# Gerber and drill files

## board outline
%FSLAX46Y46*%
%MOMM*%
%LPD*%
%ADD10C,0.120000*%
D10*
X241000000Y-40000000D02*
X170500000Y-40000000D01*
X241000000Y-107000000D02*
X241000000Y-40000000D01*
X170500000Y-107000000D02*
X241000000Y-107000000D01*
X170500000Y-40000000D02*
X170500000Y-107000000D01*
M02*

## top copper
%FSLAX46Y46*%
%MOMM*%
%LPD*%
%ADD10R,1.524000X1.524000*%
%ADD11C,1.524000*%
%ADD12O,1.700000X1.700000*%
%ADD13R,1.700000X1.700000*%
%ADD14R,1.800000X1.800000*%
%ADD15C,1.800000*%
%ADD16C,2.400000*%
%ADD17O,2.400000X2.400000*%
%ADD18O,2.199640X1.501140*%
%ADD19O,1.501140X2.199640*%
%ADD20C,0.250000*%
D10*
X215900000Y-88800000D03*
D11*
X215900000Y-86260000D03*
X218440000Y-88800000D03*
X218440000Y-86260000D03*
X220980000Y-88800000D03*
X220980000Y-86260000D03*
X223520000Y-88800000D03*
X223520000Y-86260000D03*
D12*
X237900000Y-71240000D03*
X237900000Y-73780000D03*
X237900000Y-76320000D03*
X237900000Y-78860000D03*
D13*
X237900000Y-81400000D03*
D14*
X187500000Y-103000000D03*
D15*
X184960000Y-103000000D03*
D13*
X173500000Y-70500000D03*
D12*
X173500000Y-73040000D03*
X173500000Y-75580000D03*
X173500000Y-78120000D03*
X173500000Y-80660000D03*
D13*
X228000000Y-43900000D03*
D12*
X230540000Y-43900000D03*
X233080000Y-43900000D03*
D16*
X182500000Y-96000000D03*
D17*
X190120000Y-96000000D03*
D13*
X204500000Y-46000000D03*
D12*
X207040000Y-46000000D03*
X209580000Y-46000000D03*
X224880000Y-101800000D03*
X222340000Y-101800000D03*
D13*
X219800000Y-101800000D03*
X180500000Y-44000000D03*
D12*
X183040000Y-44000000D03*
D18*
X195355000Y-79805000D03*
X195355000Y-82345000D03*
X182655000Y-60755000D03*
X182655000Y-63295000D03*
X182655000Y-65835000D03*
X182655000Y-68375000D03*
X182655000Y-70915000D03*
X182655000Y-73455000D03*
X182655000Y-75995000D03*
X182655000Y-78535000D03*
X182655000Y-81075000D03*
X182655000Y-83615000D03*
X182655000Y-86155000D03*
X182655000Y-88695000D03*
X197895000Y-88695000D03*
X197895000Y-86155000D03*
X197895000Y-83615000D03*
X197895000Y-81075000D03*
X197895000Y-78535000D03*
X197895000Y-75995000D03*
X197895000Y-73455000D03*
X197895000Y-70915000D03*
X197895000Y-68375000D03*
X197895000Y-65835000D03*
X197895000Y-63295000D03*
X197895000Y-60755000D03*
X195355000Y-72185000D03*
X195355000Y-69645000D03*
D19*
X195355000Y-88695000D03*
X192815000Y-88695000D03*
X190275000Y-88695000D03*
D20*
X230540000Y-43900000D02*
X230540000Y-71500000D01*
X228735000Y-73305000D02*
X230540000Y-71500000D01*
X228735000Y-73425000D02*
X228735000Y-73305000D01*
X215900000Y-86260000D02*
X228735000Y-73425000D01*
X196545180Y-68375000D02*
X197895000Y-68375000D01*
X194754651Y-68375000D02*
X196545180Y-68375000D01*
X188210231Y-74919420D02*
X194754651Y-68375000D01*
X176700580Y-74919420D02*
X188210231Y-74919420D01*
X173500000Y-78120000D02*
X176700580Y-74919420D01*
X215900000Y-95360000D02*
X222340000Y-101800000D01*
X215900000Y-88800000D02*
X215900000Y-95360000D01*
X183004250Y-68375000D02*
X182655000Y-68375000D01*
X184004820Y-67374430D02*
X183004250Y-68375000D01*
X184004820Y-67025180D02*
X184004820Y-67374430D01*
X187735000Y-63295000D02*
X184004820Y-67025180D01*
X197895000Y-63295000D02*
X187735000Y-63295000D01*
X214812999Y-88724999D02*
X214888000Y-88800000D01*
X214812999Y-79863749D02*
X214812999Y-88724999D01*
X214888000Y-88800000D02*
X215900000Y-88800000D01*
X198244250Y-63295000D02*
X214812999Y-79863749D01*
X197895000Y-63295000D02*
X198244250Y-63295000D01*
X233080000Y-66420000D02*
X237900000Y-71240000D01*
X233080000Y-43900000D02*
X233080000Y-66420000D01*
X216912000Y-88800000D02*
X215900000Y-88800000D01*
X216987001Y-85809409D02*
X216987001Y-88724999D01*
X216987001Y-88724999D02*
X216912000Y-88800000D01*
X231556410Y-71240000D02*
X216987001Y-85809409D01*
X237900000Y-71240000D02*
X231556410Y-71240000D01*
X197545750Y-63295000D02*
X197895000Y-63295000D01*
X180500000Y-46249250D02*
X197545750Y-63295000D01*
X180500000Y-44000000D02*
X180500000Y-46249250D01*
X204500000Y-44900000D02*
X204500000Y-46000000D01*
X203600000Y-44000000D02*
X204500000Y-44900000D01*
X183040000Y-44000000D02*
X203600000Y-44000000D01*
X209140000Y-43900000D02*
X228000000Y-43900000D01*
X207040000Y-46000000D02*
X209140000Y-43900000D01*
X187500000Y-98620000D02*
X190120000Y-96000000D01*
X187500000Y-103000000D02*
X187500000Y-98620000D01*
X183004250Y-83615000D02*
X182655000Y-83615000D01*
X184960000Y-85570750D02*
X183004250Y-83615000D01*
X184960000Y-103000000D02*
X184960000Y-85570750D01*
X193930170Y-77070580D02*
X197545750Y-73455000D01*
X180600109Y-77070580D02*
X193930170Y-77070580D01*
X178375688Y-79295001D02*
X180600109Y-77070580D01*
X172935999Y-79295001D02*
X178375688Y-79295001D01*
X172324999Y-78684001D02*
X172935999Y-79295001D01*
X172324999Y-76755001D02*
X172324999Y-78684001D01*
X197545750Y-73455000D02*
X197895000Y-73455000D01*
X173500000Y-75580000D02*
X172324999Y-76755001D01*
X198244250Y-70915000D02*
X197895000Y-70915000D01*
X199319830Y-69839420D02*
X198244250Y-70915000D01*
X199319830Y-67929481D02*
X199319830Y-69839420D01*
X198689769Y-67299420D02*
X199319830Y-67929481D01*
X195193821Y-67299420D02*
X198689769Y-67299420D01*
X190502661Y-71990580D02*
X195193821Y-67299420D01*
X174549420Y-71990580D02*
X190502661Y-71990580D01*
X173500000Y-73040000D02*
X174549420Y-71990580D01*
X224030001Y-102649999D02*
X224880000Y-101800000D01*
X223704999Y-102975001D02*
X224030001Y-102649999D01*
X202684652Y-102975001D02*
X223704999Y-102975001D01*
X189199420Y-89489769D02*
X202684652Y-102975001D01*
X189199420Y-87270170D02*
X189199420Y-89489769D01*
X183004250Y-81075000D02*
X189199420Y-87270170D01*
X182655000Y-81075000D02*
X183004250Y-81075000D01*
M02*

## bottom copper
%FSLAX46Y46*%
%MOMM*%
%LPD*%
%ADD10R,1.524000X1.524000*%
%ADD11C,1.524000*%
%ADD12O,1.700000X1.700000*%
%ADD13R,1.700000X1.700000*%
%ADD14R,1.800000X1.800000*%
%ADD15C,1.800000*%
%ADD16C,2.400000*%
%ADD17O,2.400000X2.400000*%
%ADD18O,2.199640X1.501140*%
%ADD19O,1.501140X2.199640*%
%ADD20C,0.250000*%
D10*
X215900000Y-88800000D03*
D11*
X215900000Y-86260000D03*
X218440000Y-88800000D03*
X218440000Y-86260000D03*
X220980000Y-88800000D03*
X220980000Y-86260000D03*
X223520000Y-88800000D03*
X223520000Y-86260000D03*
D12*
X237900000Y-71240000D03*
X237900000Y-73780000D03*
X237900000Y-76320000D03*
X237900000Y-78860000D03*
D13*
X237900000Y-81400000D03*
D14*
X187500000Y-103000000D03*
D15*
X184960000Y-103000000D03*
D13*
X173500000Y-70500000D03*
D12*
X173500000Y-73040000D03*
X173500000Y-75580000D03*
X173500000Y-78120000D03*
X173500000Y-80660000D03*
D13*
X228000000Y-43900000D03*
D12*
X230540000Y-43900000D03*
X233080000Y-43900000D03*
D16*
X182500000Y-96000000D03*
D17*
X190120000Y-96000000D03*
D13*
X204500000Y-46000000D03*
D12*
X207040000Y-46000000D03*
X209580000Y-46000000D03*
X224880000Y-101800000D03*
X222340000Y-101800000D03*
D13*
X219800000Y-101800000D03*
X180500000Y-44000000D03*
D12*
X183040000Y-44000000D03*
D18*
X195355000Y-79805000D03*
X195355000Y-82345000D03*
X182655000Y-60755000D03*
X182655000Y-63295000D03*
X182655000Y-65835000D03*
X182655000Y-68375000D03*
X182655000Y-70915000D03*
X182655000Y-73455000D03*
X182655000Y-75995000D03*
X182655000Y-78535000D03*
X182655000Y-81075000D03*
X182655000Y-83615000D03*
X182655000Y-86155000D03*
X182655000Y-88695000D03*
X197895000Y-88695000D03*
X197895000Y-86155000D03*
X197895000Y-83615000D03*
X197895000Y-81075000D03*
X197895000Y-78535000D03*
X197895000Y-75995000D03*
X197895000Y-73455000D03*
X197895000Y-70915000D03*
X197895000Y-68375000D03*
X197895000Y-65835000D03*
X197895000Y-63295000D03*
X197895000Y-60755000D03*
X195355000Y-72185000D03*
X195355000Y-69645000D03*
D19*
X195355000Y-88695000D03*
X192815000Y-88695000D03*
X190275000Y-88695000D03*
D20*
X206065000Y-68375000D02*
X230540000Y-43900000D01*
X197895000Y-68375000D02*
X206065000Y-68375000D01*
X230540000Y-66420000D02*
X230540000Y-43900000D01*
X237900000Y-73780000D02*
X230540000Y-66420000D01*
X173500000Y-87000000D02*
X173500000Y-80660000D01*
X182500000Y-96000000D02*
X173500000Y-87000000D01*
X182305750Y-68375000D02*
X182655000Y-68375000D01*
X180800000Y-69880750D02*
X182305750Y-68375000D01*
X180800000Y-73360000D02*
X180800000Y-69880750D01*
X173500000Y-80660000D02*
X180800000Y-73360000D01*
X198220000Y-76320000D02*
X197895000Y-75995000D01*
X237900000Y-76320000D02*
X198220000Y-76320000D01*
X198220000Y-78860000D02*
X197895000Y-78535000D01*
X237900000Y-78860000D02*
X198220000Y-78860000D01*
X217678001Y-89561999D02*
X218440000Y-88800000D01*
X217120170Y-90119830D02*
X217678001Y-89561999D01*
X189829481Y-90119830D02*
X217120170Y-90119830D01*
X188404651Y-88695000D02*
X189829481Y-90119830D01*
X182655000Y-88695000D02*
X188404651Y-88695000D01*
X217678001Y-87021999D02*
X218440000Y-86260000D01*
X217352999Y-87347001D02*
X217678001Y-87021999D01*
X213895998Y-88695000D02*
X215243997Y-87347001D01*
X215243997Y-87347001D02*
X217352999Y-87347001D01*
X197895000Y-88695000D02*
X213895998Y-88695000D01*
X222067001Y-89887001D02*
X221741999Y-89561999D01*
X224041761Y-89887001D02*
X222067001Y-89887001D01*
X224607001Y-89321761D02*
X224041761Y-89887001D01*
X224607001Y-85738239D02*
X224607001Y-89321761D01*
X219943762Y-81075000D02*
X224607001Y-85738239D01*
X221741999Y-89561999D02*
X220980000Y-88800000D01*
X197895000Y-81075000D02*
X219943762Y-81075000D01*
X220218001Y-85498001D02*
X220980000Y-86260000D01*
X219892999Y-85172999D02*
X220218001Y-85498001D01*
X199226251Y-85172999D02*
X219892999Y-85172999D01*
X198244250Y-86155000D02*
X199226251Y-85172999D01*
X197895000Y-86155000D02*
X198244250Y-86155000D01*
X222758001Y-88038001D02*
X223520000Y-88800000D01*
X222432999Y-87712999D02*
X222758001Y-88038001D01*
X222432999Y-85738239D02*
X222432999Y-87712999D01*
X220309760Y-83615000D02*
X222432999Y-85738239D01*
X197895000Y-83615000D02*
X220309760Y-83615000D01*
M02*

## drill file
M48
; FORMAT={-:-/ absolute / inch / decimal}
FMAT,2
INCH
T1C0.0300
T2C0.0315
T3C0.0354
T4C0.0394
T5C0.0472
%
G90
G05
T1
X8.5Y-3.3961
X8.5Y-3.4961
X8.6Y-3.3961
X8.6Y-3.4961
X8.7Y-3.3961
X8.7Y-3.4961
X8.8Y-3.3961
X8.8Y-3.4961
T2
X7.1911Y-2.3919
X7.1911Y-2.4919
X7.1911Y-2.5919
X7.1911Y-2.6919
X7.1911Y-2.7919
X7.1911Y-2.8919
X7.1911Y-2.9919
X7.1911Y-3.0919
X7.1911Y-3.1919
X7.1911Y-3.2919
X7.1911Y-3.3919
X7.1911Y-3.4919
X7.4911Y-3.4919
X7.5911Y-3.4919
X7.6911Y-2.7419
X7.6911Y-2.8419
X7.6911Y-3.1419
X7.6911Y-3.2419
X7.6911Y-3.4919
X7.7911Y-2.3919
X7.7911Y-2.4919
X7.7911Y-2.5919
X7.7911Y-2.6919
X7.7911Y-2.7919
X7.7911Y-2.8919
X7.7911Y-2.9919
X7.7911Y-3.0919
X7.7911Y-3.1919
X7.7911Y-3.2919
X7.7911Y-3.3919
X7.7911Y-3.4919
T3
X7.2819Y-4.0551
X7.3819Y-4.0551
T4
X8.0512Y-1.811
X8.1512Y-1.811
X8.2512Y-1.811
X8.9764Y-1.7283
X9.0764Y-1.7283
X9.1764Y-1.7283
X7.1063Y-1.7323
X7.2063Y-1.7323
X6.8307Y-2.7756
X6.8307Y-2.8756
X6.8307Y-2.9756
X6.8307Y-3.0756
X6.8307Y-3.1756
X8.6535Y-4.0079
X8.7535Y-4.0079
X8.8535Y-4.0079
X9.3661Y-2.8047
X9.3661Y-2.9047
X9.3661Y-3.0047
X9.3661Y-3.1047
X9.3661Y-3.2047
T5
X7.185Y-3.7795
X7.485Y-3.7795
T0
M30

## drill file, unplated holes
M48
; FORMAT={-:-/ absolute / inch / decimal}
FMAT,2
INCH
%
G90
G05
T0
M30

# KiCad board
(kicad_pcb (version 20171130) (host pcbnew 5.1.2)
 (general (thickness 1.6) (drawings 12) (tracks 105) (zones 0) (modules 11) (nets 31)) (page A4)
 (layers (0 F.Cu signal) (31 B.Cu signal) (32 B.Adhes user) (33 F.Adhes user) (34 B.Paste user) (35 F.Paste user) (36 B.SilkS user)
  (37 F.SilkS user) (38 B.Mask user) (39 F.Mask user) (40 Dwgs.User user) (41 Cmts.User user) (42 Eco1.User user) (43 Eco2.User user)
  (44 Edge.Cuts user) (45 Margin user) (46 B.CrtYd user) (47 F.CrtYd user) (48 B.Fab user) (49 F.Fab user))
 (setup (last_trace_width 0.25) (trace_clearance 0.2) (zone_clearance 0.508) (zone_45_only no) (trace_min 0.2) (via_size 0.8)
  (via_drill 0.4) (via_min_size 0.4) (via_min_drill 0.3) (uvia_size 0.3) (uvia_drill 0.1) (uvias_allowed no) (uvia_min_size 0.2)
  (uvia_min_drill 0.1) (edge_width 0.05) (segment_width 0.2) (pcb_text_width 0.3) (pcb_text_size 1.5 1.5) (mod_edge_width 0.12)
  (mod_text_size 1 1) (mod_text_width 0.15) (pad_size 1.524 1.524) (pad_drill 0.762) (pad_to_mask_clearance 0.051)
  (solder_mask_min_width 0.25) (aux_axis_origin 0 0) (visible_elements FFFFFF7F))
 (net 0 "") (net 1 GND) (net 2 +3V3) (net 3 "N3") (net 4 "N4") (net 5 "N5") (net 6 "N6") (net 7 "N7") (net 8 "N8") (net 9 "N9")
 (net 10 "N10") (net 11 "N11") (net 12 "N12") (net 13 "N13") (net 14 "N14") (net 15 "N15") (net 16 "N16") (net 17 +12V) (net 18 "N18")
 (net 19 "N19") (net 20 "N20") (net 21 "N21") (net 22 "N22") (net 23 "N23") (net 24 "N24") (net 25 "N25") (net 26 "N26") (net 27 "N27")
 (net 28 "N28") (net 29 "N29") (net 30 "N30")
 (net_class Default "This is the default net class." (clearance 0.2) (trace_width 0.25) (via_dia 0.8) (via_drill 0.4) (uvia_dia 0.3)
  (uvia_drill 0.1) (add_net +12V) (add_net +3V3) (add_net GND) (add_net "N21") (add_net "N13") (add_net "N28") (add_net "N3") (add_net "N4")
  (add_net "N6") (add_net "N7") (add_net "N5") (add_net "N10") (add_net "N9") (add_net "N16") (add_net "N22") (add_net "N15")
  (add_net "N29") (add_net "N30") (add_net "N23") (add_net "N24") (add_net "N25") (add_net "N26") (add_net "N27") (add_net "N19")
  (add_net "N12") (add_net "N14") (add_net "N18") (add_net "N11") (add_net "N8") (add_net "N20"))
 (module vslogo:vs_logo (layer B.Cu) (at 206.325 86.925 180)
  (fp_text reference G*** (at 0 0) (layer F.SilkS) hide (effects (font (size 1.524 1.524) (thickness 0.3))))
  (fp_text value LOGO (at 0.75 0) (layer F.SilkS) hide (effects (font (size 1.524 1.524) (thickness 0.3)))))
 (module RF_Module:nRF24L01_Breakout (layer F.Cu) (at 215.9 88.8 90)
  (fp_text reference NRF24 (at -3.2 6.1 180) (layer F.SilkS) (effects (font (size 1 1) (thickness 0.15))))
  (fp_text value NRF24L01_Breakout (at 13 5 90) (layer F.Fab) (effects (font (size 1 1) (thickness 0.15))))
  (pad 1 thru_hole rect (at 0 0 90) (size 1.524 1.524) (drill 0.762) (layers *.Cu *.Mask) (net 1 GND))
  (pad 2 thru_hole circle (at 2.54 0 90) (size 1.524 1.524) (drill 0.762) (layers *.Cu *.Mask) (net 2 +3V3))
  (pad 3 thru_hole circle (at 0 2.54 90) (size 1.524 1.524) (drill 0.762) (layers *.Cu *.Mask) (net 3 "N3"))
  (pad 4 thru_hole circle (at 2.54 2.54 90) (size 1.524 1.524) (drill 0.762) (layers *.Cu *.Mask) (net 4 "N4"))
  (pad 5 thru_hole circle (at 0 5.08 90) (size 1.524 1.524) (drill 0.762) (layers *.Cu *.Mask) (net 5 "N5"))
  (pad 6 thru_hole circle (at 2.54 5.08 90) (size 1.524 1.524) (drill 0.762) (layers *.Cu *.Mask) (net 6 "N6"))
  (pad 7 thru_hole circle (at 0 7.62 90) (size 1.524 1.524) (drill 0.762) (layers *.Cu *.Mask) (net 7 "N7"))
  (pad 8 thru_hole circle (at 2.54 7.62 90) (size 1.524 1.524) (drill 0.762) (layers *.Cu *.Mask) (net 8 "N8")))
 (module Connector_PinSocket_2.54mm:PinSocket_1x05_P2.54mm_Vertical (layer F.Cu) (at 237.9 81.4 180)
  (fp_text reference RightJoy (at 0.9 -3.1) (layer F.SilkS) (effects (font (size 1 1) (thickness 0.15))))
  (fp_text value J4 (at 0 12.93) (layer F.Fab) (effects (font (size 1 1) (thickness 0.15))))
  (pad 5 thru_hole oval (at 0 10.16 180) (size 1.7 1.7) (drill 1) (layers *.Cu *.Mask) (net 1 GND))
  (pad 4 thru_hole oval (at 0 7.62 180) (size 1.7 1.7) (drill 1) (layers *.Cu *.Mask) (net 2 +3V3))
  (pad 3 thru_hole oval (at 0 5.08 180) (size 1.7 1.7) (drill 1) (layers *.Cu *.Mask) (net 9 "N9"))
  (pad 2 thru_hole oval (at 0 2.54 180) (size 1.7 1.7) (drill 1) (layers *.Cu *.Mask) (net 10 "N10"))
  (pad 1 thru_hole rect (at 0 0 180) (size 1.7 1.7) (drill 1) (layers *.Cu *.Mask) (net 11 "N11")))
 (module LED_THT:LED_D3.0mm (layer F.Cu) (at 187.5 103 180)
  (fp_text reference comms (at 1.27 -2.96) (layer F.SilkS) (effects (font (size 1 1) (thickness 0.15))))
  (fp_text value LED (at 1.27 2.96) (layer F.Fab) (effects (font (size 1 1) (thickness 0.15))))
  (pad 1 thru_hole rect (at 0 0 180) (size 1.8 1.8) (drill 0.9) (layers *.Cu *.Mask) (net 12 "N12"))
  (pad 2 thru_hole circle (at 2.54 0 180) (size 1.8 1.8) (drill 0.9) (layers *.Cu *.Mask) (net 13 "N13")))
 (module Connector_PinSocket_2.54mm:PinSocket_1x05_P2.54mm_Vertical (layer F.Cu) (at 173.5 70.5)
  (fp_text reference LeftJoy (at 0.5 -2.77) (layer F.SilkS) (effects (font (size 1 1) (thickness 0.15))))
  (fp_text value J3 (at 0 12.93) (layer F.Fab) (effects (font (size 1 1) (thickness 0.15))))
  (pad 1 thru_hole rect (at 0 0) (size 1.7 1.7) (drill 1) (layers *.Cu *.Mask) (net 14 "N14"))
  (pad 2 thru_hole oval (at 0 2.54) (size 1.7 1.7) (drill 1) (layers *.Cu *.Mask) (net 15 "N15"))
  (pad 3 thru_hole oval (at 0 5.08) (size 1.7 1.7) (drill 1) (layers *.Cu *.Mask) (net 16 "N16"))
  (pad 4 thru_hole oval (at 0 7.62) (size 1.7 1.7) (drill 1) (layers *.Cu *.Mask) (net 2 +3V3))
  (pad 5 thru_hole oval (at 0 10.16) (size 1.7 1.7) (drill 1) (layers *.Cu *.Mask) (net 1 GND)))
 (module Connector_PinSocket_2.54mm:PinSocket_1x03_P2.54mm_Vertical (layer F.Cu) (at 228 43.9 90)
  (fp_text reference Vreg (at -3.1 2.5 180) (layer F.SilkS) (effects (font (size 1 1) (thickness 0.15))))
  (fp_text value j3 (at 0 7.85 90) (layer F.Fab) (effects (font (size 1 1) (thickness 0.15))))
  (pad 1 thru_hole rect (at 0 0 90) (size 1.7 1.7) (drill 1) (layers *.Cu *.Mask) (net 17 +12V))
  (pad 2 thru_hole oval (at 0 2.54 90) (size 1.7 1.7) (drill 1) (layers *.Cu *.Mask) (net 2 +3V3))
  (pad 3 thru_hole oval (at 0 5.08 90) (size 1.7 1.7) (drill 1) (layers *.Cu *.Mask) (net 1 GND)))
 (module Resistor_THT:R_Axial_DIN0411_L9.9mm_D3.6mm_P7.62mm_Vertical (layer F.Cu) (at 182.5 96)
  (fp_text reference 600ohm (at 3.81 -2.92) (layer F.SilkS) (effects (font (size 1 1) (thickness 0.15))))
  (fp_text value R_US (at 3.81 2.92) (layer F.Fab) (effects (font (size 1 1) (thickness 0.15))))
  (pad 1 thru_hole circle (at 0 0) (size 2.4 2.4) (drill 1.2) (layers *.Cu *.Mask) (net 1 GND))
  (pad 2 thru_hole oval (at 7.62 0) (size 2.4 2.4) (drill 1.2) (layers *.Cu *.Mask) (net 12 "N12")))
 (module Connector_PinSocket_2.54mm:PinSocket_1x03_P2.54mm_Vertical (layer F.Cu) (at 204.5 46 90)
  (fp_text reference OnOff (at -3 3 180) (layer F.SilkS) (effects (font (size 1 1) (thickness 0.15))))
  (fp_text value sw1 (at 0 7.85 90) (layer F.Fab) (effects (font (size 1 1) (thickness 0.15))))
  (pad 1 thru_hole rect (at 0 0 90) (size 1.7 1.7) (drill 1) (layers *.Cu *.Mask) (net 17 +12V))
  (pad 2 thru_hole oval (at 0 2.54 90) (size 1.7 1.7) (drill 1) (layers *.Cu *.Mask) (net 17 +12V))
  (pad 3 thru_hole oval (at 0 5.08 90) (size 1.7 1.7) (drill 1) (layers *.Cu *.Mask) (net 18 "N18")))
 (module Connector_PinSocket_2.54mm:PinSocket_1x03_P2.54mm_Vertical (layer F.Cu) (at 219.8 101.8 90)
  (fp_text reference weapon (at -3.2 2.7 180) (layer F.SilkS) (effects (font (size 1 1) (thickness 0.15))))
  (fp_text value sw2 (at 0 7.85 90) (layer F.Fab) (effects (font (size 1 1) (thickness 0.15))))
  (pad 3 thru_hole oval (at 0 5.08 90) (size 1.7 1.7) (drill 1) (layers *.Cu *.Mask) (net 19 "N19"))
  (pad 2 thru_hole oval (at 0 2.54 90) (size 1.7 1.7) (drill 1) (layers *.Cu *.Mask) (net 1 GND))
  (pad 1 thru_hole rect (at 0 0 90) (size 1.7 1.7) (drill 1) (layers *.Cu *.Mask) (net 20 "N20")))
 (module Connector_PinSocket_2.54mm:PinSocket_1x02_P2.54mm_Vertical (layer F.Cu) (at 180.5 44 90)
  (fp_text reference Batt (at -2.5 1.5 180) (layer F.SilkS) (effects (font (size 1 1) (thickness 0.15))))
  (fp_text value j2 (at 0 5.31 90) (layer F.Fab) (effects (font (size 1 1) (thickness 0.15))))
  (pad 1 thru_hole rect (at 0 0 90) (size 1.7 1.7) (drill 1) (layers *.Cu *.Mask) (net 1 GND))
  (pad 2 thru_hole oval (at 0 2.54 90) (size 1.7 1.7) (drill 1) (layers *.Cu *.Mask) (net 17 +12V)))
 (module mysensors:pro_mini (layer F.Cu) (at 190.275 74.725 270)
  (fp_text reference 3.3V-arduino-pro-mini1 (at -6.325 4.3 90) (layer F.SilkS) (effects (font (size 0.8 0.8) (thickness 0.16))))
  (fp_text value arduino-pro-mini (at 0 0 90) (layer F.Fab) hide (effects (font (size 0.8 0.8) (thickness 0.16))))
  (pad 28 thru_hole oval (at 5.08 -5.08 270) (size 1.50114 2.19964) (drill 0.8001) (layers *.Cu *.Mask F.SilkS))
  (pad 27 thru_hole oval (at 7.62 -5.08 270) (size 1.50114 2.19964) (drill 0.8001) (layers *.Cu *.Mask F.SilkS))
  (pad 1 thru_hole oval (at -13.97 7.62 270) (size 1.50114 2.19964) (drill 0.8001) (layers *.Cu *.Mask F.SilkS) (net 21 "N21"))
  (pad 2 thru_hole oval (at -11.43 7.62 270) (size 1.50114 2.19964) (drill 0.8001) (layers *.Cu *.Mask F.SilkS) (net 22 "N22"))
  (pad 3 thru_hole oval (at -8.89 7.62 270) (size 1.50114 2.19964) (drill 0.8001) (layers *.Cu *.Mask F.SilkS) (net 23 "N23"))
  (pad 4 thru_hole oval (at -6.35 7.62 270) (size 1.50114 2.19964) (drill 0.8001) (layers *.Cu *.Mask F.SilkS) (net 1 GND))
  (pad 5 thru_hole oval (at -3.81 7.62 270) (size 1.50114 2.19964) (drill 0.8001) (layers *.Cu *.Mask F.SilkS) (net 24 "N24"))
  (pad 6 thru_hole oval (at -1.27 7.62 270) (size 1.50114 2.19964) (drill 0.8001) (layers *.Cu *.Mask F.SilkS) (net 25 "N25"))
  (pad 7 thru_hole oval (at 1.27 7.62 270) (size 1.50114 2.19964) (drill 0.8001) (layers *.Cu *.Mask F.SilkS) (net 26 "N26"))
  (pad 8 thru_hole oval (at 3.81 7.62 270) (size 1.50114 2.19964) (drill 0.8001) (layers *.Cu *.Mask F.SilkS) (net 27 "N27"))
  (pad 9 thru_hole oval (at 6.35 7.62 270) (size 1.50114 2.19964) (drill 0.8001) (layers *.Cu *.Mask F.SilkS) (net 19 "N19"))
  (pad 10 thru_hole oval (at 8.89 7.62 270) (size 1.50114 2.19964) (drill 0.8001) (layers *.Cu *.Mask F.SilkS) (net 13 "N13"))
  (pad 11 thru_hole oval (at 11.43 7.62 270) (size 1.50114 2.19964) (drill 0.8001) (layers *.Cu *.Mask F.SilkS) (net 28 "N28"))
  (pad 12 thru_hole oval (at 13.97 7.62 270) (size 1.50114 2.19964) (drill 0.8001) (layers *.Cu *.Mask F.SilkS) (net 3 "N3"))
  (pad 13 thru_hole oval (at 13.97 -7.62 270) (size 1.50114 2.19964) (drill 0.8001) (layers *.Cu *.Mask F.SilkS) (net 4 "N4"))
  (pad 14 thru_hole oval (at 11.43 -7.62 270) (size 1.50114 2.19964) (drill 0.8001) (layers *.Cu *.Mask F.SilkS) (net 6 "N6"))
  (pad 15 thru_hole oval (at 8.89 -7.62 270) (size 1.50114 2.19964) (drill 0.8001) (layers *.Cu *.Mask F.SilkS) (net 7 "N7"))
  (pad 16 thru_hole oval (at 6.35 -7.62 270) (size 1.50114 2.19964) (drill 0.8001) (layers *.Cu *.Mask F.SilkS) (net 5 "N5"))
  (pad 17 thru_hole oval (at 3.81 -7.62 270) (size 1.50114 2.19964) (drill 0.8001) (layers *.Cu *.Mask F.SilkS) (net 10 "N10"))
  (pad 18 thru_hole oval (at 1.27 -7.62 270) (size 1.50114 2.19964) (drill 0.8001) (layers *.Cu *.Mask F.SilkS) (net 9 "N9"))
  (pad 19 thru_hole oval (at -1.27 -7.62 270) (size 1.50114 2.19964) (drill 0.8001) (layers *.Cu *.Mask F.SilkS) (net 16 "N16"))
  (pad 20 thru_hole oval (at -3.81 -7.62 270) (size 1.50114 2.19964) (drill 0.8001) (layers *.Cu *.Mask F.SilkS) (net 15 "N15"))
  (pad 21 thru_hole oval (at -6.35 -7.62 270) (size 1.50114 2.19964) (drill 0.8001) (layers *.Cu *.Mask F.SilkS) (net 2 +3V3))
  (pad 22 thru_hole oval (at -8.89 -7.62 270) (size 1.50114 2.19964) (drill 0.8001) (layers *.Cu *.Mask F.SilkS) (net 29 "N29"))
  (pad 23 thru_hole oval (at -11.43 -7.62 270) (size 1.50114 2.19964) (drill 0.8001) (layers *.Cu *.Mask F.SilkS) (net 1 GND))
  (pad 24 thru_hole oval (at -13.97 -7.62 270) (size 1.50114 2.19964) (drill 0.8001) (layers *.Cu *.Mask F.SilkS) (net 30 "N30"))
  (pad 25 thru_hole oval (at -2.54 -5.08 270) (size 1.50114 2.19964) (drill 0.8001) (layers *.Cu *.Mask F.SilkS))
  (pad 26 thru_hole oval (at -5.08 -5.08 270) (size 1.50114 2.19964) (drill 0.8001) (layers *.Cu *.Mask F.SilkS))
  (pad 27 thru_hole oval (at 13.97 -5.08 270) (size 2.19964 1.50114) (drill 0.8001) (layers *.Cu *.Mask F.SilkS))
  (pad 28 thru_hole oval (at 13.97 -2.54 270) (size 2.19964 1.50114) (drill 0.8001) (layers *.Cu *.Mask F.SilkS))
  (pad 29 thru_hole oval (at 13.97 0 270) (size 2.19964 1.50114) (drill 0.8001) (layers *.Cu *.Mask F.SilkS)))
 (gr_line (start 241 40) (end 170.5 40) (layer Edge.Cuts) (width 0.12))
 (gr_line (start 241 107) (end 241 40) (layer Edge.Cuts) (width 0.12))
 (gr_line (start 170.5 107) (end 241 107) (layer Edge.Cuts) (width 0.12))
 (gr_line (start 170.5 40) (end 170.5 107) (layer Edge.Cuts) (width 0.12))
 (segment (start 230.54 43.9) (end 230.54 71.5) (width 0.25) (layer F.Cu) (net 2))
 (segment (start 228.735 73.305) (end 230.54 71.5) (width 0.25) (layer F.Cu) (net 2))
 (segment (start 228.735 73.425) (end 228.735 73.305) (width 0.25) (layer F.Cu) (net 2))
 (segment (start 215.9 86.26) (end 228.735 73.425) (width 0.25) (layer F.Cu) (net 2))
 (segment (start 206.065 68.375) (end 230.54 43.9) (width 0.25) (layer B.Cu) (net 2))
 (segment (start 197.895 68.375) (end 206.065 68.375) (width 0.25) (layer B.Cu) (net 2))
 (segment (start 230.54 66.42) (end 230.54 43.9) (width 0.25) (layer B.Cu) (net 2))
 (segment (start 237.9 73.78) (end 230.54 66.42) (width 0.25) (layer B.Cu) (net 2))
 (segment (start 196.54518 68.375) (end 197.895 68.375) (width 0.25) (layer F.Cu) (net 2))
 (segment (start 194.754651 68.375) (end 196.54518 68.375) (width 0.25) (layer F.Cu) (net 2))
 (segment (start 188.210231 74.91942) (end 194.754651 68.375) (width 0.25) (layer F.Cu) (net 2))
 (segment (start 176.70058 74.91942) (end 188.210231 74.91942) (width 0.25) (layer F.Cu) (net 2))
 (segment (start 173.5 78.12) (end 176.70058 74.91942) (width 0.25) (layer F.Cu) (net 2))
 (segment (start 215.9 95.36) (end 222.34 101.8) (width 0.25) (layer F.Cu) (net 1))
 (segment (start 215.9 88.8) (end 215.9 95.36) (width 0.25) (layer F.Cu) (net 1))
 (segment (start 183.00425 68.375) (end 182.655 68.375) (width 0.25) (layer F.Cu) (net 1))
 (segment (start 184.00482 67.37443) (end 183.00425 68.375) (width 0.25) (layer F.Cu) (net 1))
 (segment (start 184.00482 67.02518) (end 184.00482 67.37443) (width 0.25) (layer F.Cu) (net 1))
 (segment (start 187.735 63.295) (end 184.00482 67.02518) (width 0.25) (layer F.Cu) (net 1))
 (segment (start 197.895 63.295) (end 187.735 63.295) (width 0.25) (layer F.Cu) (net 1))
 (segment (start 214.812999 88.724999) (end 214.888 88.8) (width 0.25) (layer F.Cu) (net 1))
 (segment (start 214.812999 79.863749) (end 214.812999 88.724999) (width 0.25) (layer F.Cu) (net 1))
 (segment (start 214.888 88.8) (end 215.9 88.8) (width 0.25) (layer F.Cu) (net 1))
 (segment (start 198.24425 63.295) (end 214.812999 79.863749) (width 0.25) (layer F.Cu) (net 1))
 (segment (start 197.895 63.295) (end 198.24425 63.295) (width 0.25) (layer F.Cu) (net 1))
 (segment (start 233.08 66.42) (end 237.9 71.24) (width 0.25) (layer F.Cu) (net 1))
 (segment (start 233.08 43.9) (end 233.08 66.42) (width 0.25) (layer F.Cu) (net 1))
 (segment (start 216.912 88.8) (end 215.9 88.8) (width 0.25) (layer F.Cu) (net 1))
 (segment (start 216.987001 85.809409) (end 216.987001 88.724999) (width 0.25) (layer F.Cu) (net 1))
 (segment (start 216.987001 88.724999) (end 216.912 88.8) (width 0.25) (layer F.Cu) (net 1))
 (segment (start 231.55641 71.24) (end 216.987001 85.809409) (width 0.25) (layer F.Cu) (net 1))
 (segment (start 237.9 71.24) (end 231.55641 71.24) (width 0.25) (layer F.Cu) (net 1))
 (segment (start 173.5 87) (end 173.5 80.66) (width 0.25) (layer B.Cu) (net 1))
 (segment (start 182.5 96) (end 173.5 87) (width 0.25) (layer B.Cu) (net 1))
 (segment (start 182.30575 68.375) (end 182.655 68.375) (width 0.25) (layer B.Cu) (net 1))
 (segment (start 180.8 69.88075) (end 182.30575 68.375) (width 0.25) (layer B.Cu) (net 1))
 (segment (start 180.8 73.36) (end 180.8 69.88075) (width 0.25) (layer B.Cu) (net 1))
 (segment (start 173.5 80.66) (end 180.8 73.36) (width 0.25) (layer B.Cu) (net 1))
 (segment (start 197.54575 63.295) (end 197.895 63.295) (width 0.25) (layer F.Cu) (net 1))
 (segment (start 180.5 46.24925) (end 197.54575 63.295) (width 0.25) (layer F.Cu) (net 1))
 (segment (start 180.5 44) (end 180.5 46.24925) (width 0.25) (layer F.Cu) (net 1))
 (segment (start 204.5 44.9) (end 204.5 46) (width 0.25) (layer F.Cu) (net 17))
 (segment (start 203.6 44) (end 204.5 44.9) (width 0.25) (layer F.Cu) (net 17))
 (segment (start 183.04 44) (end 203.6 44) (width 0.25) (layer F.Cu) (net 17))
 (segment (start 209.14 43.9) (end 228 43.9) (width 0.25) (layer F.Cu) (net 17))
 (segment (start 207.04 46) (end 209.14 43.9) (width 0.25) (layer F.Cu) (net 17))
 (segment (start 187.5 98.62) (end 190.12 96) (width 0.25) (layer F.Cu) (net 12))
 (segment (start 187.5 103) (end 187.5 98.62) (width 0.25) (layer F.Cu) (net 12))
 (segment (start 183.00425 83.615) (end 182.655 83.615) (width 0.25) (layer F.Cu) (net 13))
 (segment (start 184.96 85.57075) (end 183.00425 83.615) (width 0.25) (layer F.Cu) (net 13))
 (segment (start 184.96 103) (end 184.96 85.57075) (width 0.25) (layer F.Cu) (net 13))
 (segment (start 193.93017 77.07058) (end 197.54575 73.455) (width 0.25) (layer F.Cu) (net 16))
 (segment (start 180.600109 77.07058) (end 193.93017 77.07058) (width 0.25) (layer F.Cu) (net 16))
 (segment (start 178.375688 79.295001) (end 180.600109 77.07058) (width 0.25) (layer F.Cu) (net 16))
 (segment (start 172.935999 79.295001) (end 178.375688 79.295001) (width 0.25) (layer F.Cu) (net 16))
 (segment (start 172.324999 78.684001) (end 172.935999 79.295001) (width 0.25) (layer F.Cu) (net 16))
 (segment (start 172.324999 76.755001) (end 172.324999 78.684001) (width 0.25) (layer F.Cu) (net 16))
 (segment (start 197.54575 73.455) (end 197.895 73.455) (width 0.25) (layer F.Cu) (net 16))
 (segment (start 173.5 75.58) (end 172.324999 76.755001) (width 0.25) (layer F.Cu) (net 16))
 (segment (start 198.24425 70.915) (end 197.895 70.915) (width 0.25) (layer F.Cu) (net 15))
 (segment (start 199.31983 69.83942) (end 198.24425 70.915) (width 0.25) (layer F.Cu) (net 15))
 (segment (start 199.31983 67.929481) (end 199.31983 69.83942) (width 0.25) (layer F.Cu) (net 15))
 (segment (start 198.689769 67.29942) (end 199.31983 67.929481) (width 0.25) (layer F.Cu) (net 15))
 (segment (start 195.193821 67.29942) (end 198.689769 67.29942) (width 0.25) (layer F.Cu) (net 15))
 (segment (start 190.502661 71.99058) (end 195.193821 67.29942) (width 0.25) (layer F.Cu) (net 15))
 (segment (start 174.54942 71.99058) (end 190.502661 71.99058) (width 0.25) (layer F.Cu) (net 15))
 (segment (start 173.5 73.04) (end 174.54942 71.99058) (width 0.25) (layer F.Cu) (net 15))
 (segment (start 198.22 76.32) (end 197.895 75.995) (width 0.25) (layer B.Cu) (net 9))
 (segment (start 237.9 76.32) (end 198.22 76.32) (width 0.25) (layer B.Cu) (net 9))
 (segment (start 198.22 78.86) (end 197.895 78.535) (width 0.25) (layer B.Cu) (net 10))
 (segment (start 237.9 78.86) (end 198.22 78.86) (width 0.25) (layer B.Cu) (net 10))
 (segment (start 217.678001 89.561999) (end 218.44 88.8) (width 0.25) (layer B.Cu) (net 3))
 (segment (start 217.12017 90.11983) (end 217.678001 89.561999) (width 0.25) (layer B.Cu) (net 3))
 (segment (start 189.829481 90.11983) (end 217.12017 90.11983) (width 0.25) (layer B.Cu) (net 3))
 (segment (start 188.404651 88.695) (end 189.829481 90.11983) (width 0.25) (layer B.Cu) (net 3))
 (segment (start 182.655 88.695) (end 188.404651 88.695) (width 0.25) (layer B.Cu) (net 3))
 (segment (start 217.678001 87.021999) (end 218.44 86.26) (width 0.25) (layer B.Cu) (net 4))
 (segment (start 217.352999 87.347001) (end 217.678001 87.021999) (width 0.25) (layer B.Cu) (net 4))
 (segment (start 213.895998 88.695) (end 215.243997 87.347001) (width 0.25) (layer B.Cu) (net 4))
 (segment (start 215.243997 87.347001) (end 217.352999 87.347001) (width 0.25) (layer B.Cu) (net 4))
 (segment (start 197.895 88.695) (end 213.895998 88.695) (width 0.25) (layer B.Cu) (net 4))
 (segment (start 222.067001 89.887001) (end 221.741999 89.561999) (width 0.25) (layer B.Cu) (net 5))
 (segment (start 224.041761 89.887001) (end 222.067001 89.887001) (width 0.25) (layer B.Cu) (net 5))
 (segment (start 224.607001 89.321761) (end 224.041761 89.887001) (width 0.25) (layer B.Cu) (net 5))
 (segment (start 224.607001 85.738239) (end 224.607001 89.321761) (width 0.25) (layer B.Cu) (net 5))
 (segment (start 219.943762 81.075) (end 224.607001 85.738239) (width 0.25) (layer B.Cu) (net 5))
 (segment (start 221.741999 89.561999) (end 220.98 88.8) (width 0.25) (layer B.Cu) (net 5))
 (segment (start 197.895 81.075) (end 219.943762 81.075) (width 0.25) (layer B.Cu) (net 5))
 (segment (start 220.218001 85.498001) (end 220.98 86.26) (width 0.25) (layer B.Cu) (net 6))
 (segment (start 219.892999 85.172999) (end 220.218001 85.498001) (width 0.25) (layer B.Cu) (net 6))
 (segment (start 199.226251 85.172999) (end 219.892999 85.172999) (width 0.25) (layer B.Cu) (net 6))
 (segment (start 198.24425 86.155) (end 199.226251 85.172999) (width 0.25) (layer B.Cu) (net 6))
 (segment (start 197.895 86.155) (end 198.24425 86.155) (width 0.25) (layer B.Cu) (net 6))
 (segment (start 222.758001 88.038001) (end 223.52 88.8) (width 0.25) (layer B.Cu) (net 7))
 (segment (start 222.432999 87.712999) (end 222.758001 88.038001) (width 0.25) (layer B.Cu) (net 7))
 (segment (start 222.432999 85.738239) (end 222.432999 87.712999) (width 0.25) (layer B.Cu) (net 7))
 (segment (start 220.30976 83.615) (end 222.432999 85.738239) (width 0.25) (layer B.Cu) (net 7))
 (segment (start 197.895 83.615) (end 220.30976 83.615) (width 0.25) (layer B.Cu) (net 7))
 (segment (start 224.030001 102.649999) (end 224.88 101.8) (width 0.25) (layer F.Cu) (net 19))
 (segment (start 223.704999 102.975001) (end 224.030001 102.649999) (width 0.25) (layer F.Cu) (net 19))
 (segment (start 202.684652 102.975001) (end 223.704999 102.975001) (width 0.25) (layer F.Cu) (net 19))
 (segment (start 189.19942 89.489769) (end 202.684652 102.975001) (width 0.25) (layer F.Cu) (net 19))
 (segment (start 189.19942 87.27017) (end 189.19942 89.489769) (width 0.25) (layer F.Cu) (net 19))
 (segment (start 183.00425 81.075) (end 189.19942 87.27017) (width 0.25) (layer F.Cu) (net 19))
 (segment (start 182.655 81.075) (end 183.00425 81.075) (width 0.25) (layer F.Cu) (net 19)))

